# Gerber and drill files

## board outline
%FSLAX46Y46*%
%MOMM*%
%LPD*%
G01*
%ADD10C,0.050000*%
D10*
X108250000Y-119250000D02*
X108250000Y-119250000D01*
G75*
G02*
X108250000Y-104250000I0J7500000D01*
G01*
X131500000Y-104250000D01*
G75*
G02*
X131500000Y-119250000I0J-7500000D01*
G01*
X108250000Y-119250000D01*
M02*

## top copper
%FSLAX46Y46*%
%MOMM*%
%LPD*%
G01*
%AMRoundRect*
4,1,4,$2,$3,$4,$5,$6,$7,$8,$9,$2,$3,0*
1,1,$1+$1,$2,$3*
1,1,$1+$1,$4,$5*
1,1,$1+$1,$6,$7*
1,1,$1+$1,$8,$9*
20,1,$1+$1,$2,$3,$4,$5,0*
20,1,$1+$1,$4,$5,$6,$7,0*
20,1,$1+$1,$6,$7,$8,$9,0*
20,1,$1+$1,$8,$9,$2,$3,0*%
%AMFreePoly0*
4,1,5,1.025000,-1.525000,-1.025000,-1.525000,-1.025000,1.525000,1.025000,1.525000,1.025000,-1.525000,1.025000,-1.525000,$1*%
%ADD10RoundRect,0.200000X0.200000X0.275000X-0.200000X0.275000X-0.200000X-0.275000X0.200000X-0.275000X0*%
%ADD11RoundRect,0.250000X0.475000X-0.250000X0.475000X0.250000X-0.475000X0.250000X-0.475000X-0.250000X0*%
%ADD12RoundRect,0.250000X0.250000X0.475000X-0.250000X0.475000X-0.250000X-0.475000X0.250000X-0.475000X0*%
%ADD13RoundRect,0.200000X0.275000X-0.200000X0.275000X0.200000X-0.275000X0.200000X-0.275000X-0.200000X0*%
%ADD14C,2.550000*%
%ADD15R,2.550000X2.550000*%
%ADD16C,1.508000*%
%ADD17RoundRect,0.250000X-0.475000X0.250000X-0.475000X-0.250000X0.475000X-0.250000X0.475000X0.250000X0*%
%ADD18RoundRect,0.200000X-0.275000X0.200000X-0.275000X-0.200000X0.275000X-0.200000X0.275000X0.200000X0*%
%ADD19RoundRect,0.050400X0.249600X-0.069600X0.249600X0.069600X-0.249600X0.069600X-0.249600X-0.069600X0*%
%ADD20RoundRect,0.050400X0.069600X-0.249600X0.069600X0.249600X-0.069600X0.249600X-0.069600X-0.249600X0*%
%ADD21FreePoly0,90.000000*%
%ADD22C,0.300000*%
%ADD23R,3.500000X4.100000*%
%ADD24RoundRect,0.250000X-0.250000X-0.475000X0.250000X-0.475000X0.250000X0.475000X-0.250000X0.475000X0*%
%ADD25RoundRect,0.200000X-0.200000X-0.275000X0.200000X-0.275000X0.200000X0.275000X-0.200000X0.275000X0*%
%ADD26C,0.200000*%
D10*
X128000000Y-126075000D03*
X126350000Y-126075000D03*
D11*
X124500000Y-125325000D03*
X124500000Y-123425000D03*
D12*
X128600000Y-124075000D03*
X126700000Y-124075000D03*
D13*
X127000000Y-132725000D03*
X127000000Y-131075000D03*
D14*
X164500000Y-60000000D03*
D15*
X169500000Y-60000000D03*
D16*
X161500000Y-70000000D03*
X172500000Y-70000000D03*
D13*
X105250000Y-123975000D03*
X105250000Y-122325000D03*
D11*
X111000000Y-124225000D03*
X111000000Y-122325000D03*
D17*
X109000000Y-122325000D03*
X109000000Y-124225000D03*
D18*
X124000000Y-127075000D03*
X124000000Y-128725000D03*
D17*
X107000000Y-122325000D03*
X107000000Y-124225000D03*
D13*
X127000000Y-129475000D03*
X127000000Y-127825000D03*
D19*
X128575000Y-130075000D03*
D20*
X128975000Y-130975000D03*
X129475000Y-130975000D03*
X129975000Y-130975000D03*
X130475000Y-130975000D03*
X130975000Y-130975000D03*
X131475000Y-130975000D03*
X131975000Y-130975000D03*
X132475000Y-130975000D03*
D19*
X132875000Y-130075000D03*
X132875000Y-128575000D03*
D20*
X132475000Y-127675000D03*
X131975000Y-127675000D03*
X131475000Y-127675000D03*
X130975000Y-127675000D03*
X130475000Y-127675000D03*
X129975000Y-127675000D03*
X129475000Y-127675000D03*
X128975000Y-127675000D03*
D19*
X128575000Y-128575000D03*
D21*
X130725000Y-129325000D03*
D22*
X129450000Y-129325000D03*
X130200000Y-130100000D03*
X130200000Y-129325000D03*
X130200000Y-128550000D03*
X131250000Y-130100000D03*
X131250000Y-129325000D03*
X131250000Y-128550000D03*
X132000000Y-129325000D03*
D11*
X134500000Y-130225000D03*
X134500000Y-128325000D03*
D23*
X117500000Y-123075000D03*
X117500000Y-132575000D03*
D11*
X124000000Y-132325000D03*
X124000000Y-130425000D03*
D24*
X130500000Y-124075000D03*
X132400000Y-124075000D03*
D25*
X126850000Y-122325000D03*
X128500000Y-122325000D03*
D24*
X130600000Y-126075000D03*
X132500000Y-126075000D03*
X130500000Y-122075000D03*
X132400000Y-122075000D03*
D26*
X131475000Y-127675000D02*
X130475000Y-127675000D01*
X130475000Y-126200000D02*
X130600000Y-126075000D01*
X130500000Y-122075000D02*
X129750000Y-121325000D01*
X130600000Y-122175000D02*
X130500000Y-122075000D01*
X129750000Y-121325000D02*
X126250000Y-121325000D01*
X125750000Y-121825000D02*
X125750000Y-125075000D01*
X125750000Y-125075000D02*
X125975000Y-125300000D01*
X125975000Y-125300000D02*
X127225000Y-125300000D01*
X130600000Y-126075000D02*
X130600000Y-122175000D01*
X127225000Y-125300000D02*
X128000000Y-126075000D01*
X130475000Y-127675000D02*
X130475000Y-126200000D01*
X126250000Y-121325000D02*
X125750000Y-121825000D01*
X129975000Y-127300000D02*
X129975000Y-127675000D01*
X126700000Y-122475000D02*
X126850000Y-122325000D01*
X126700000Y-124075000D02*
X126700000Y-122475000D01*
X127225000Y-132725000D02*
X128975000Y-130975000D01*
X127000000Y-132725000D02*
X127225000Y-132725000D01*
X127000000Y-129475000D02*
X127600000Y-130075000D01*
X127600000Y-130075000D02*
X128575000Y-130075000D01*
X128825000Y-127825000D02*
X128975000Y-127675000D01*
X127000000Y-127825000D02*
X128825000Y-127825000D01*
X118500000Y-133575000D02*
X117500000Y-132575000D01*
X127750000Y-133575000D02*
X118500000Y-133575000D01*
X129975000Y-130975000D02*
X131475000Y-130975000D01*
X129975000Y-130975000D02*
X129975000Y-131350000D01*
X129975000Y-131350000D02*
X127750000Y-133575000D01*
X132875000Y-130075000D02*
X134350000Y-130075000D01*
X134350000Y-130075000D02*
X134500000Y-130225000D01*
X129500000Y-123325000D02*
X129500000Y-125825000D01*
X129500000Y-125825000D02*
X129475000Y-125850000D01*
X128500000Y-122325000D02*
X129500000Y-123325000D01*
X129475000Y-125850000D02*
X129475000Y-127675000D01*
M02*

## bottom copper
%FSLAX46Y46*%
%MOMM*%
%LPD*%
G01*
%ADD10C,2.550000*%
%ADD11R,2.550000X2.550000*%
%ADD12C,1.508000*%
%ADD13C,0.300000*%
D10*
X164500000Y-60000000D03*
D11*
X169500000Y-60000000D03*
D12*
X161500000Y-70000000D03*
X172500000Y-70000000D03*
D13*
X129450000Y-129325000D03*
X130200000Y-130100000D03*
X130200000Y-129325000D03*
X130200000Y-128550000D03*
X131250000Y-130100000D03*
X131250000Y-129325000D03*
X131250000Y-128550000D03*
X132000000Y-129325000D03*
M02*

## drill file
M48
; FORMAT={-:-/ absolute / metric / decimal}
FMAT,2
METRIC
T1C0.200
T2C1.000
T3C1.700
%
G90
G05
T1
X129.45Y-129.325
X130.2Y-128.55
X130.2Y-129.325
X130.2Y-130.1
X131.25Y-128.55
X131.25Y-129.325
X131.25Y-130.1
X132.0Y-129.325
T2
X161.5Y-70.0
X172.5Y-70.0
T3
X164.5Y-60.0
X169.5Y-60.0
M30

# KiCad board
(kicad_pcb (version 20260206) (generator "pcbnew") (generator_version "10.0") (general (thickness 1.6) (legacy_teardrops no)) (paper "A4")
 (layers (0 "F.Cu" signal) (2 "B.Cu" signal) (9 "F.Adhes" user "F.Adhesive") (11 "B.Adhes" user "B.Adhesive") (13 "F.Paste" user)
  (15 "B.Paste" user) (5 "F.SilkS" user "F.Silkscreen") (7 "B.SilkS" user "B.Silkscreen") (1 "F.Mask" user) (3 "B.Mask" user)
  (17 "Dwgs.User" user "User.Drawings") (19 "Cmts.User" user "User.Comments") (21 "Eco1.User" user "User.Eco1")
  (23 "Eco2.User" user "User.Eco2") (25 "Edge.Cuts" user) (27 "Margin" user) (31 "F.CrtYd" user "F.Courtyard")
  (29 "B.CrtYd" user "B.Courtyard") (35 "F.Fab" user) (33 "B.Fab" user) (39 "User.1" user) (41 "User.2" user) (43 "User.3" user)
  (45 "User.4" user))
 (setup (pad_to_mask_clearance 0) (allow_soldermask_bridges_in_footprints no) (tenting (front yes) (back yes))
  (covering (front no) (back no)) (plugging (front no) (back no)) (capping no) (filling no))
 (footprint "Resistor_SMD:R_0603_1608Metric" (layer "F.Cu") (at 127.175 126.075 180)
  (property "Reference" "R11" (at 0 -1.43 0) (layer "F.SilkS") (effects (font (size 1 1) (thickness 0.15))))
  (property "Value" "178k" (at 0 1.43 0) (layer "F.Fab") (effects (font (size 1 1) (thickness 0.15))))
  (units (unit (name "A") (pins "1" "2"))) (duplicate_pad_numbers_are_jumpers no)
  (pad "1" smd roundrect (at -0.825 0 180) (size 0.8 0.95) (layers "F.Cu" "F.Mask" "F.Paste") (roundrect_rratio 0.25) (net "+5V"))
  (pad "2" smd roundrect (at 0.825 0 180) (size 0.8 0.95) (layers "F.Cu" "F.Mask" "F.Paste") (roundrect_rratio 0.25) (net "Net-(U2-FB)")))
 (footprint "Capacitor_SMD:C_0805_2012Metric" (layer "F.Cu") (at 124.5 124.375 90)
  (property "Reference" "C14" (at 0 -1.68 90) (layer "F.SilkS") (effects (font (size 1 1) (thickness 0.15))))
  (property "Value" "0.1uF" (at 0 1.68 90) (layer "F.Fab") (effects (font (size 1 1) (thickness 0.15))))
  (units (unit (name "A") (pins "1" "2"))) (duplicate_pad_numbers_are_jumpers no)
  (pad "1" smd roundrect (at -0.95 0 90) (size 1 1.45) (layers "F.Cu" "F.Mask" "F.Paste") (roundrect_rratio 0.25) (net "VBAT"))
  (pad "2" smd roundrect (at 0.95 0 90) (size 1 1.45) (layers "F.Cu" "F.Mask" "F.Paste") (roundrect_rratio 0.25) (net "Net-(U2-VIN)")))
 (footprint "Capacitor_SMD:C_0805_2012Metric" (layer "F.Cu") (at 127.65 124.075 180)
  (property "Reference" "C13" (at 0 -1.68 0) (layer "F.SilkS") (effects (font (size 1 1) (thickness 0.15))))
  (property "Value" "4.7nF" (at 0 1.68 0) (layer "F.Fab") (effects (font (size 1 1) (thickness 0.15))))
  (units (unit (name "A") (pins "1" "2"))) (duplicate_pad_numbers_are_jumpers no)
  (pad "1" smd roundrect (at -0.95 0 180) (size 1 1.45) (layers "F.Cu" "F.Mask" "F.Paste") (roundrect_rratio 0.25) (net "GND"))
  (pad "2" smd roundrect (at 0.95 0 180) (size 1 1.45) (layers "F.Cu" "F.Mask" "F.Paste") (roundrect_rratio 0.25) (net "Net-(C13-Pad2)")))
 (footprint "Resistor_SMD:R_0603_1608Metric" (layer "F.Cu") (at 127 131.9 90)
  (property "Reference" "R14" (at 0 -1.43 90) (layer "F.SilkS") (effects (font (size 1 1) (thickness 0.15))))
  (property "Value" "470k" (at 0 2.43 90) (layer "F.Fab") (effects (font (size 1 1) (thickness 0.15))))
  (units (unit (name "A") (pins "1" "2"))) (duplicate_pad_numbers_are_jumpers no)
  (pad "1" smd roundrect (at -0.825 0 90) (size 0.8 0.95) (layers "F.Cu" "F.Mask" "F.Paste") (roundrect_rratio 0.25) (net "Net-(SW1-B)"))
  (pad "2" smd roundrect (at 0.825 0 90) (size 0.8 0.95) (layers "F.Cu" "F.Mask" "F.Paste") (roundrect_rratio 0.25) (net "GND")))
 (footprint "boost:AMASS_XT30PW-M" (layer "F.Cu") (at 167 70 180)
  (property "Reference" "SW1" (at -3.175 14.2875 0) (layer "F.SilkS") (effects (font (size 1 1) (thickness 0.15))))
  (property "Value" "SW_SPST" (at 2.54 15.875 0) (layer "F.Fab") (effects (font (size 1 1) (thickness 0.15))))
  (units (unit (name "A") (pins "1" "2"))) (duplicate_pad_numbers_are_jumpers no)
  (pad "N" thru_hole circle (at 2.5 10 180) (size 2.55 2.55) (drill 1.7) (layers "*.Cu" "*.Mask") (remove_unused_layers no)
   (solder_mask_margin 0.102))
  (pad "P" thru_hole rect (at -2.5 10 180) (size 2.55 2.55) (drill 1.7) (layers "*.Cu" "*.Mask") (remove_unused_layers no)
   (solder_mask_margin 0.102))
  (pad "S1" thru_hole circle (at 5.5 0 180) (size 1.508 1.508) (drill 1) (layers "*.Cu" "*.Mask") (remove_unused_layers no)
   (solder_mask_margin 0.102))
  (pad "S2" thru_hole circle (at -5.5 0 180) (size 1.508 1.508) (drill 1) (layers "*.Cu" "*.Mask") (remove_unused_layers no)
   (solder_mask_margin 0.102)))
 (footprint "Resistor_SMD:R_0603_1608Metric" (layer "F.Cu") (at 105.25 123.15 90)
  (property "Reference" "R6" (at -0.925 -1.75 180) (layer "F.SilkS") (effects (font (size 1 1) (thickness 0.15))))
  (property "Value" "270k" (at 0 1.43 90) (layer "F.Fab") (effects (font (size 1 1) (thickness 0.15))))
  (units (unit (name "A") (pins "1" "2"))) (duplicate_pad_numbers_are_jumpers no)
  (pad "1" smd roundrect (at -0.825 0 90) (size 0.8 0.95) (layers "F.Cu" "F.Mask" "F.Paste") (roundrect_rratio 0.25) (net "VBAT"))
  (pad "2" smd roundrect (at 0.825 0 90) (size 0.8 0.95) (layers "F.Cu" "F.Mask" "F.Paste") (roundrect_rratio 0.25) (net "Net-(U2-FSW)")))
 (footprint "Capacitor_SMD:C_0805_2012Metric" (layer "F.Cu") (at 111 123.275 90)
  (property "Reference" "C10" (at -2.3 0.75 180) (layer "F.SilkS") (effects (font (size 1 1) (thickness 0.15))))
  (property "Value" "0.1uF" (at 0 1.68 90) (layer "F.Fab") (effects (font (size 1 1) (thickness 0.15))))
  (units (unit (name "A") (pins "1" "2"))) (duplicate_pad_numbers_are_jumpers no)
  (pad "1" smd roundrect (at -0.95 0 90) (size 1 1.45) (layers "F.Cu" "F.Mask" "F.Paste") (roundrect_rratio 0.25) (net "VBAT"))
  (pad "2" smd roundrect (at 0.95 0 90) (size 1 1.45) (layers "F.Cu" "F.Mask" "F.Paste") (roundrect_rratio 0.25) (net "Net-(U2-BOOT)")))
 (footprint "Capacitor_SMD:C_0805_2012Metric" (layer "F.Cu") (at 109 123.275 -90)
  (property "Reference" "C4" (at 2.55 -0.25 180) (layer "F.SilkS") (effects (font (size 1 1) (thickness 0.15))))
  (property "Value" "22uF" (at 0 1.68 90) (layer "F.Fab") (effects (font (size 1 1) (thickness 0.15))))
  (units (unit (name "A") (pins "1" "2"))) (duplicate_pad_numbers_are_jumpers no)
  (pad "1" smd roundrect (at -0.95 0 270) (size 1 1.45) (layers "F.Cu" "F.Mask" "F.Paste") (roundrect_rratio 0.25) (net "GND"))
  (pad "2" smd roundrect (at 0.95 0 270) (size 1 1.45) (layers "F.Cu" "F.Mask" "F.Paste") (roundrect_rratio 0.25) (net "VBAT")))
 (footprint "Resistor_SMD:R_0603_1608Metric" (layer "F.Cu") (at 124 127.9 -90)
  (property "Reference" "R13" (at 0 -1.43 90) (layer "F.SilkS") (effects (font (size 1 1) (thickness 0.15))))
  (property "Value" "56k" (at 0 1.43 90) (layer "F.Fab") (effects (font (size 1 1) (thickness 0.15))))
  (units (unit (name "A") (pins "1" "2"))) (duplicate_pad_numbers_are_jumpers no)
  (pad "1" smd roundrect (at -0.825 0 270) (size 0.8 0.95) (layers "F.Cu" "F.Mask" "F.Paste") (roundrect_rratio 0.25) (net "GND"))
  (pad "2" smd roundrect (at 0.825 0 270) (size 0.8 0.95) (layers "F.Cu" "F.Mask" "F.Paste") (roundrect_rratio 0.25) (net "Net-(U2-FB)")))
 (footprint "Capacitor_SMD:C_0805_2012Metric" (layer "F.Cu") (at 107 123.275 -90)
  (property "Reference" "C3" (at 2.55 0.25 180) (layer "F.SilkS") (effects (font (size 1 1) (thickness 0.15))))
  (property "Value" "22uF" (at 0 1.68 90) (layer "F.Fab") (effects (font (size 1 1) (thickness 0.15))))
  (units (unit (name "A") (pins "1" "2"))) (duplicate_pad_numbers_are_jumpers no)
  (pad "1" smd roundrect (at -0.95 0 270) (size 1 1.45) (layers "F.Cu" "F.Mask" "F.Paste") (roundrect_rratio 0.25) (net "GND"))
  (pad "2" smd roundrect (at 0.95 0 270) (size 1 1.45) (layers "F.Cu" "F.Mask" "F.Paste") (roundrect_rratio 0.25) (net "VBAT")))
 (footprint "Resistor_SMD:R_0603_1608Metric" (layer "F.Cu") (at 127 128.65 90)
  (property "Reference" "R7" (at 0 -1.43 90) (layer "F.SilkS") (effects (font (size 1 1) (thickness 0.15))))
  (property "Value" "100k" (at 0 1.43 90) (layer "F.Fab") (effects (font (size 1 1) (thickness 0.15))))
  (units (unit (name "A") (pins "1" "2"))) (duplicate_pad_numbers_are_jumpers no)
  (pad "1" smd roundrect (at -0.825 0 90) (size 0.8 0.95) (layers "F.Cu" "F.Mask" "F.Paste") (roundrect_rratio 0.25) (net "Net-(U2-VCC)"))
  (pad "2" smd roundrect (at 0.825 0 90) (size 0.8 0.95) (layers "F.Cu" "F.Mask" "F.Paste") (roundrect_rratio 0.25) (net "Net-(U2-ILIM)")))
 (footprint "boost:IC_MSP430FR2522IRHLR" (layer "F.Cu") (at 130.725 129.325 90)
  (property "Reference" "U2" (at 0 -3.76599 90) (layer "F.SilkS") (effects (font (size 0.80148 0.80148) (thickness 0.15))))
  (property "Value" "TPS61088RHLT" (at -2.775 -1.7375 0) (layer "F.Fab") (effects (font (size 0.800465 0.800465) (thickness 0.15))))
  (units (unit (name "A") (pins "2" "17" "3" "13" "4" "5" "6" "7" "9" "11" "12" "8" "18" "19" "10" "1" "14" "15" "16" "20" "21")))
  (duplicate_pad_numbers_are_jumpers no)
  (pad "1" smd roundrect (at -0.75 -2.15 90) (size 0.24 0.6) (layers "F.Cu" "F.Mask" "F.Paste") (roundrect_rratio 0.21) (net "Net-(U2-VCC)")
   (solder_mask_margin 0.102))
  (pad "2" smd roundrect (at -1.65 -1.75 90) (size 0.6 0.24) (layers "F.Cu" "F.Mask" "F.Paste") (roundrect_rratio 0.21) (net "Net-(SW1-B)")
   (solder_mask_margin 0.102))
  (pad "3" smd roundrect (at -1.65 -1.25 90) (size 0.6 0.24) (layers "F.Cu" "F.Mask" "F.Paste") (roundrect_rratio 0.21) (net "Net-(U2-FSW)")
   (solder_mask_margin 0.102))
  (pad "4" smd roundrect (at -1.65 -0.75 90) (size 0.6 0.24) (layers "F.Cu" "F.Mask" "F.Paste") (roundrect_rratio 0.21)
   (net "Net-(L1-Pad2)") (solder_mask_margin 0.102))
  (pad "5" smd roundrect (at -1.65 -0.25 90) (size 0.6 0.24) (layers "F.Cu" "F.Mask" "F.Paste") (roundrect_rratio 0.21)
   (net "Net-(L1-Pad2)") (solder_mask_margin 0.102))
  (pad "6" smd roundrect (at -1.65 0.25 90) (size 0.6 0.24) (layers "F.Cu" "F.Mask" "F.Paste") (roundrect_rratio 0.21) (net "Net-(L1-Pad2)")
   (solder_mask_margin 0.102))
  (pad "7" smd roundrect (at -1.65 0.75 90) (size 0.6 0.24) (layers "F.Cu" "F.Mask" "F.Paste") (roundrect_rratio 0.21) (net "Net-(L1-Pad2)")
   (solder_mask_margin 0.102))
  (pad "8" smd roundrect (at -1.65 1.25 90) (size 0.6 0.24) (layers "F.Cu" "F.Mask" "F.Paste") (roundrect_rratio 0.21) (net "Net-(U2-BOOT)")
   (solder_mask_margin 0.102))
  (pad "9" smd roundrect (at -1.65 1.75 90) (size 0.6 0.24) (layers "F.Cu" "F.Mask" "F.Paste") (roundrect_rratio 0.21) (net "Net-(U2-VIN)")
   (solder_mask_margin 0.102))
  (pad "10" smd roundrect (at -0.75 2.15 90) (size 0.24 0.6) (layers "F.Cu" "F.Mask" "F.Paste") (roundrect_rratio 0.21) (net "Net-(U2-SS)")
   (solder_mask_margin 0.102))
  (pad "11" smd roundrect (at 0.75 2.15 90) (size 0.24 0.6) (layers "F.Cu" "F.Mask" "F.Paste") (roundrect_rratio 0.21)
   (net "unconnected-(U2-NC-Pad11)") (solder_mask_margin 0.102))
  (pad "12" smd roundrect (at 1.65 1.75 90) (size 0.6 0.24) (layers "F.Cu" "F.Mask" "F.Paste") (roundrect_rratio 0.21)
   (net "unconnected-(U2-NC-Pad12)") (solder_mask_margin 0.102))
  (pad "13" smd roundrect (at 1.65 1.25 90) (size 0.6 0.24) (layers "F.Cu" "F.Mask" "F.Paste") (roundrect_rratio 0.21) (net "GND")
   (solder_mask_margin 0.102))
  (pad "14" smd roundrect (at 1.65 0.75 90) (size 0.6 0.24) (layers "F.Cu" "F.Mask" "F.Paste") (roundrect_rratio 0.21) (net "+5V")
   (solder_mask_margin 0.102))
  (pad "15" smd roundrect (at 1.65 0.25 90) (size 0.6 0.24) (layers "F.Cu" "F.Mask" "F.Paste") (roundrect_rratio 0.21) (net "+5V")
   (solder_mask_margin 0.102))
  (pad "16" smd roundrect (at 1.65 -0.25 90) (size 0.6 0.24) (layers "F.Cu" "F.Mask" "F.Paste") (roundrect_rratio 0.21) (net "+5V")
   (solder_mask_margin 0.102))
  (pad "17" smd roundrect (at 1.65 -0.75 90) (size 0.6 0.24) (layers "F.Cu" "F.Mask" "F.Paste") (roundrect_rratio 0.21) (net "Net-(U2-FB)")
   (solder_mask_margin 0.102))
  (pad "18" smd roundrect (at 1.65 -1.25 90) (size 0.6 0.24) (layers "F.Cu" "F.Mask" "F.Paste") (roundrect_rratio 0.21)
   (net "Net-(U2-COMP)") (solder_mask_margin 0.102))
  (pad "19" smd roundrect (at 1.65 -1.75 90) (size 0.6 0.24) (layers "F.Cu" "F.Mask" "F.Paste") (roundrect_rratio 0.21)
   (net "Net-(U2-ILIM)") (solder_mask_margin 0.102))
  (pad "20" smd roundrect (at 0.75 -2.15 90) (size 0.24 0.6) (layers "F.Cu" "F.Mask" "F.Paste") (roundrect_rratio 0.21) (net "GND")
   (solder_mask_margin 0.102))
  (pad "21" smd custom (at 0 0 90) (size 2.05 3.05) (layers "F.Cu" "F.Mask") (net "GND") (solder_mask_margin 0.102)
   (options (clearance outline) (anchor rect)) (primitives))
  (pad "22" thru_hole circle (at 0 -1.275 90) (size 0.3 0.3) (drill 0.2) (layers "*.Cu" "*.Mask") (remove_unused_layers no)
   (solder_mask_margin 0.102))
  (pad "23" thru_hole circle (at -0.775 -0.525 90) (size 0.3 0.3) (drill 0.2) (layers "*.Cu" "*.Mask") (remove_unused_layers no)
   (solder_mask_margin 0.102))
  (pad "24" thru_hole circle (at 0 -0.525 90) (size 0.3 0.3) (drill 0.2) (layers "*.Cu" "*.Mask") (remove_unused_layers no)
   (solder_mask_margin 0.102))
  (pad "25" thru_hole circle (at 0.775 -0.525 90) (size 0.3 0.3) (drill 0.2) (layers "*.Cu" "*.Mask") (remove_unused_layers no)
   (solder_mask_margin 0.102))
  (pad "26" thru_hole circle (at -0.775 0.525 90) (size 0.3 0.3) (drill 0.2) (layers "*.Cu" "*.Mask") (remove_unused_layers no)
   (solder_mask_margin 0.102))
  (pad "27" thru_hole circle (at 0 0.525 90) (size 0.3 0.3) (drill 0.2) (layers "*.Cu" "*.Mask") (remove_unused_layers no)
   (solder_mask_margin 0.102))
  (pad "28" thru_hole circle (at 0.775 0.525 90) (size 0.3 0.3) (drill 0.2) (layers "*.Cu" "*.Mask") (remove_unused_layers no)
   (solder_mask_margin 0.102))
  (pad "29" thru_hole circle (at 0 1.275 90) (size 0.3 0.3) (drill 0.2) (layers "*.Cu" "*.Mask") (remove_unused_layers no)
   (solder_mask_margin 0.102)))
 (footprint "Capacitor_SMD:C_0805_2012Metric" (layer "F.Cu") (at 134.5 129.275 90)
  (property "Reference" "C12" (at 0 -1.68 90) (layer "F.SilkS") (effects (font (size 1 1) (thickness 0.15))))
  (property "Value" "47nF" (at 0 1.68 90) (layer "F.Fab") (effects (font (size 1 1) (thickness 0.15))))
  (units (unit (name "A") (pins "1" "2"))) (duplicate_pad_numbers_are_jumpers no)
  (pad "1" smd roundrect (at -0.95 0 90) (size 1 1.45) (layers "F.Cu" "F.Mask" "F.Paste") (roundrect_rratio 0.25) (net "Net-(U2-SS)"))
  (pad "2" smd roundrect (at 0.95 0 90) (size 1 1.45) (layers "F.Cu" "F.Mask" "F.Paste") (roundrect_rratio 0.25) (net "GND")))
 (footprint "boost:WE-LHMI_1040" (layer "F.Cu") (at 117.5 127.825 -90)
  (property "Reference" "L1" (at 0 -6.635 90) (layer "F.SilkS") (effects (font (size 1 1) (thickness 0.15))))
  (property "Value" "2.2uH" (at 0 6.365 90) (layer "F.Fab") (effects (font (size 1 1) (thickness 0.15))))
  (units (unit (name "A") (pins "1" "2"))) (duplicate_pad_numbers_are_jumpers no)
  (pad "1" smd rect (at -4.75 0 270) (size 4.1 3.5) (layers "F.Cu" "F.Mask" "F.Paste") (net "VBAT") (solder_mask_margin 0.102))
  (pad "2" smd rect (at 4.75 0 270) (size 4.1 3.5) (layers "F.Cu" "F.Mask" "F.Paste") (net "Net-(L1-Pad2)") (solder_mask_margin 0.102))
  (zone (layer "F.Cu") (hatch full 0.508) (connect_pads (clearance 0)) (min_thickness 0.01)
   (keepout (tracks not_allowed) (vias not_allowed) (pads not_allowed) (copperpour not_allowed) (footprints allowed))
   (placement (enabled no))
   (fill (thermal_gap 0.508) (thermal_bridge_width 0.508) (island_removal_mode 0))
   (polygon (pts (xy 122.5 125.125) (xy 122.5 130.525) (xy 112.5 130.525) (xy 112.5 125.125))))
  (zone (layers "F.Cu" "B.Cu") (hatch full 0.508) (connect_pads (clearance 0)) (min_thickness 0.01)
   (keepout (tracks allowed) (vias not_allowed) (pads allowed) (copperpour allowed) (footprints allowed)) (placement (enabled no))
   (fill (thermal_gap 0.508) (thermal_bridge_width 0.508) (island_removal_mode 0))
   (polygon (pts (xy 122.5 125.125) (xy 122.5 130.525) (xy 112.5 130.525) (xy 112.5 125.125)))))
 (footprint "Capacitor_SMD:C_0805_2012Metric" (layer "F.Cu") (at 124 131.375 90)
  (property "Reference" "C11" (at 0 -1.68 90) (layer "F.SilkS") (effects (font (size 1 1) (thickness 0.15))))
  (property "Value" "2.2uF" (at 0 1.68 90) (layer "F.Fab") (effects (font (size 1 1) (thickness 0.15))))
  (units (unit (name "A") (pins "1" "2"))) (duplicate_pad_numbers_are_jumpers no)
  (pad "1" smd roundrect (at -0.95 0 90) (size 1 1.45) (layers "F.Cu" "F.Mask" "F.Paste") (roundrect_rratio 0.25) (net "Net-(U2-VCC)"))
  (pad "2" smd roundrect (at 0.95 0 90) (size 1 1.45) (layers "F.Cu" "F.Mask" "F.Paste") (roundrect_rratio 0.25) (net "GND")))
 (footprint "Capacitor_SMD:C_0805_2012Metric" (layer "F.Cu") (at 131.45 124.075)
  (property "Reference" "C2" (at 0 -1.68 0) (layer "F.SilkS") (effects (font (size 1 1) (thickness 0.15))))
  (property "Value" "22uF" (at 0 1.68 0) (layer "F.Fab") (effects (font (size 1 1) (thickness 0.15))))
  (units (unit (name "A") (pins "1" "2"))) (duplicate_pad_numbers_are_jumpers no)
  (pad "1" smd roundrect (at -0.95 0) (size 1 1.45) (layers "F.Cu" "F.Mask" "F.Paste") (roundrect_rratio 0.25) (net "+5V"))
  (pad "2" smd roundrect (at 0.95 0) (size 1 1.45) (layers "F.Cu" "F.Mask" "F.Paste") (roundrect_rratio 0.25) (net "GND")))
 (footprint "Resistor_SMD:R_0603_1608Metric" (layer "F.Cu") (at 127.675 122.325)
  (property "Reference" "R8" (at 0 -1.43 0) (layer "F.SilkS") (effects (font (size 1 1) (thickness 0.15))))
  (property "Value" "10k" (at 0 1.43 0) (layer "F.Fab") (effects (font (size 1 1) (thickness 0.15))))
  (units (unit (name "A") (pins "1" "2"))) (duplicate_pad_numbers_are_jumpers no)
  (pad "1" smd roundrect (at -0.825 0) (size 0.8 0.95) (layers "F.Cu" "F.Mask" "F.Paste") (roundrect_rratio 0.25) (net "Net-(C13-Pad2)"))
  (pad "2" smd roundrect (at 0.825 0) (size 0.8 0.95) (layers "F.Cu" "F.Mask" "F.Paste") (roundrect_rratio 0.25) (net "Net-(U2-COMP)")))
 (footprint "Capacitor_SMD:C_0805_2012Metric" (layer "F.Cu") (at 131.55 126.075)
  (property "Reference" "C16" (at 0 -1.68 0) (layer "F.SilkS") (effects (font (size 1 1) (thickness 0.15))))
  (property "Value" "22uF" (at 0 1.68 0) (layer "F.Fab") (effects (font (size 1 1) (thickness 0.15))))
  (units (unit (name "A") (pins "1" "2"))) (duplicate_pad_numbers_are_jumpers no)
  (pad "1" smd roundrect (at -0.95 0) (size 1 1.45) (layers "F.Cu" "F.Mask" "F.Paste") (roundrect_rratio 0.25) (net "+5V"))
  (pad "2" smd roundrect (at 0.95 0) (size 1 1.45) (layers "F.Cu" "F.Mask" "F.Paste") (roundrect_rratio 0.25) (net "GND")))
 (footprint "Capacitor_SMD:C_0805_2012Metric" (layer "F.Cu") (at 131.45 122.075)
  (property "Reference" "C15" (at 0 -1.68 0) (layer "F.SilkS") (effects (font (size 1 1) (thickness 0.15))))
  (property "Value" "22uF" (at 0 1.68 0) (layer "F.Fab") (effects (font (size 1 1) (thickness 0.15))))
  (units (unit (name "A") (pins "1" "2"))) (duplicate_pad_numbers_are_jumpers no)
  (pad "1" smd roundrect (at -0.95 0) (size 1 1.45) (layers "F.Cu" "F.Mask" "F.Paste") (roundrect_rratio 0.25) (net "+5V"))
  (pad "2" smd roundrect (at 0.95 0) (size 1 1.45) (layers "F.Cu" "F.Mask" "F.Paste") (roundrect_rratio 0.25) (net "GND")))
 (gr_rect (start 100.75 104.25) (end 139 119.25) (radius 7.5) (stroke (width 0.05) (type default)) (fill no) (layer "Edge.Cuts"))
 (segment (start 131.475 127.675) (end 130.475 127.675) (width 0.2) (layer "F.Cu") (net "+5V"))
 (segment (start 130.475 126.2) (end 130.6 126.075) (width 0.2) (layer "F.Cu") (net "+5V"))
 (segment (start 130.5 122.075) (end 129.75 121.325) (width 0.2) (layer "F.Cu") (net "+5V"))
 (segment (start 130.6 122.175) (end 130.5 122.075) (width 0.2) (layer "F.Cu") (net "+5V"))
 (segment (start 129.75 121.325) (end 126.25 121.325) (width 0.2) (layer "F.Cu") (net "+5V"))
 (segment (start 125.75 121.825) (end 125.75 125.075) (width 0.2) (layer "F.Cu") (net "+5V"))
 (segment (start 125.75 125.075) (end 125.975 125.3) (width 0.2) (layer "F.Cu") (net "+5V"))
 (segment (start 125.975 125.3) (end 127.225 125.3) (width 0.2) (layer "F.Cu") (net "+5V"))
 (segment (start 130.6 126.075) (end 130.6 122.175) (width 0.2) (layer "F.Cu") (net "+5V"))
 (segment (start 127.225 125.3) (end 128 126.075) (width 0.2) (layer "F.Cu") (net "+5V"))
 (segment (start 130.475 127.675) (end 130.475 126.2) (width 0.2) (layer "F.Cu") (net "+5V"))
 (segment (start 126.25 121.325) (end 125.75 121.825) (width 0.2) (layer "F.Cu") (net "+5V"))
 (segment (start 129.975 127.3) (end 129.975 127.675) (width 0.2) (layer "F.Cu") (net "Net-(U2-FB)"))
 (segment (start 126.7 122.475) (end 126.85 122.325) (width 0.2) (layer "F.Cu") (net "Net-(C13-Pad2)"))
 (segment (start 126.7 124.075) (end 126.7 122.475) (width 0.2) (layer "F.Cu") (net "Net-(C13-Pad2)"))
 (segment (start 127.225 132.725) (end 128.975 130.975) (width 0.2) (layer "F.Cu") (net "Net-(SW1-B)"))
 (segment (start 127 132.725) (end 127.225 132.725) (width 0.2) (layer "F.Cu") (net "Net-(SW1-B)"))
 (segment (start 127 129.475) (end 127.6 130.075) (width 0.2) (layer "F.Cu") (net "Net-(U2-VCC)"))
 (segment (start 127.6 130.075) (end 128.575 130.075) (width 0.2) (layer "F.Cu") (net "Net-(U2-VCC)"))
 (segment (start 128.825 127.825) (end 128.975 127.675) (width 0.2) (layer "F.Cu") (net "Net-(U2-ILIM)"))
 (segment (start 127 127.825) (end 128.825 127.825) (width 0.2) (layer "F.Cu") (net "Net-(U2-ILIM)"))
 (segment (start 118.5 133.575) (end 117.5 132.575) (width 0.2) (layer "F.Cu") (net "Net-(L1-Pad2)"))
 (segment (start 127.75 133.575) (end 118.5 133.575) (width 0.2) (layer "F.Cu") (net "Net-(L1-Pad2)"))
 (segment (start 129.975 130.975) (end 131.475 130.975) (width 0.2) (layer "F.Cu") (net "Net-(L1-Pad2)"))
 (segment (start 129.975 130.975) (end 129.975 131.35) (width 0.2) (layer "F.Cu") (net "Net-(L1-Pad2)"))
 (segment (start 129.975 131.35) (end 127.75 133.575) (width 0.2) (layer "F.Cu") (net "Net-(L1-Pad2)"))
 (segment (start 132.875 130.075) (end 134.35 130.075) (width 0.2) (layer "F.Cu") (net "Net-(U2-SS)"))
 (segment (start 134.35 130.075) (end 134.5 130.225) (width 0.2) (layer "F.Cu") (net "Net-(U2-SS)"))
 (segment (start 129.5 123.325) (end 129.5 125.825) (width 0.2) (layer "F.Cu") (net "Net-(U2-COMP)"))
 (segment (start 129.5 125.825) (end 129.475 125.85) (width 0.2) (layer "F.Cu") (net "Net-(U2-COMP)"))
 (segment (start 128.5 122.325) (end 129.5 123.325) (width 0.2) (layer "F.Cu") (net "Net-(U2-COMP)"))
 (segment (start 129.475 125.85) (end 129.475 127.675) (width 0.2) (layer "F.Cu") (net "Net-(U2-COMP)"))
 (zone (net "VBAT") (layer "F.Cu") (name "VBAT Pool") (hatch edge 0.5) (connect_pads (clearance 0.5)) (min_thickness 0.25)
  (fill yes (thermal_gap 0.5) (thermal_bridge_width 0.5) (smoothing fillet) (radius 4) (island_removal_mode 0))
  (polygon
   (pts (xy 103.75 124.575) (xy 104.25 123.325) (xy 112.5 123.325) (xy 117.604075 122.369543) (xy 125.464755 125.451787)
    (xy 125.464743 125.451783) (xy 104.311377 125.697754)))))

